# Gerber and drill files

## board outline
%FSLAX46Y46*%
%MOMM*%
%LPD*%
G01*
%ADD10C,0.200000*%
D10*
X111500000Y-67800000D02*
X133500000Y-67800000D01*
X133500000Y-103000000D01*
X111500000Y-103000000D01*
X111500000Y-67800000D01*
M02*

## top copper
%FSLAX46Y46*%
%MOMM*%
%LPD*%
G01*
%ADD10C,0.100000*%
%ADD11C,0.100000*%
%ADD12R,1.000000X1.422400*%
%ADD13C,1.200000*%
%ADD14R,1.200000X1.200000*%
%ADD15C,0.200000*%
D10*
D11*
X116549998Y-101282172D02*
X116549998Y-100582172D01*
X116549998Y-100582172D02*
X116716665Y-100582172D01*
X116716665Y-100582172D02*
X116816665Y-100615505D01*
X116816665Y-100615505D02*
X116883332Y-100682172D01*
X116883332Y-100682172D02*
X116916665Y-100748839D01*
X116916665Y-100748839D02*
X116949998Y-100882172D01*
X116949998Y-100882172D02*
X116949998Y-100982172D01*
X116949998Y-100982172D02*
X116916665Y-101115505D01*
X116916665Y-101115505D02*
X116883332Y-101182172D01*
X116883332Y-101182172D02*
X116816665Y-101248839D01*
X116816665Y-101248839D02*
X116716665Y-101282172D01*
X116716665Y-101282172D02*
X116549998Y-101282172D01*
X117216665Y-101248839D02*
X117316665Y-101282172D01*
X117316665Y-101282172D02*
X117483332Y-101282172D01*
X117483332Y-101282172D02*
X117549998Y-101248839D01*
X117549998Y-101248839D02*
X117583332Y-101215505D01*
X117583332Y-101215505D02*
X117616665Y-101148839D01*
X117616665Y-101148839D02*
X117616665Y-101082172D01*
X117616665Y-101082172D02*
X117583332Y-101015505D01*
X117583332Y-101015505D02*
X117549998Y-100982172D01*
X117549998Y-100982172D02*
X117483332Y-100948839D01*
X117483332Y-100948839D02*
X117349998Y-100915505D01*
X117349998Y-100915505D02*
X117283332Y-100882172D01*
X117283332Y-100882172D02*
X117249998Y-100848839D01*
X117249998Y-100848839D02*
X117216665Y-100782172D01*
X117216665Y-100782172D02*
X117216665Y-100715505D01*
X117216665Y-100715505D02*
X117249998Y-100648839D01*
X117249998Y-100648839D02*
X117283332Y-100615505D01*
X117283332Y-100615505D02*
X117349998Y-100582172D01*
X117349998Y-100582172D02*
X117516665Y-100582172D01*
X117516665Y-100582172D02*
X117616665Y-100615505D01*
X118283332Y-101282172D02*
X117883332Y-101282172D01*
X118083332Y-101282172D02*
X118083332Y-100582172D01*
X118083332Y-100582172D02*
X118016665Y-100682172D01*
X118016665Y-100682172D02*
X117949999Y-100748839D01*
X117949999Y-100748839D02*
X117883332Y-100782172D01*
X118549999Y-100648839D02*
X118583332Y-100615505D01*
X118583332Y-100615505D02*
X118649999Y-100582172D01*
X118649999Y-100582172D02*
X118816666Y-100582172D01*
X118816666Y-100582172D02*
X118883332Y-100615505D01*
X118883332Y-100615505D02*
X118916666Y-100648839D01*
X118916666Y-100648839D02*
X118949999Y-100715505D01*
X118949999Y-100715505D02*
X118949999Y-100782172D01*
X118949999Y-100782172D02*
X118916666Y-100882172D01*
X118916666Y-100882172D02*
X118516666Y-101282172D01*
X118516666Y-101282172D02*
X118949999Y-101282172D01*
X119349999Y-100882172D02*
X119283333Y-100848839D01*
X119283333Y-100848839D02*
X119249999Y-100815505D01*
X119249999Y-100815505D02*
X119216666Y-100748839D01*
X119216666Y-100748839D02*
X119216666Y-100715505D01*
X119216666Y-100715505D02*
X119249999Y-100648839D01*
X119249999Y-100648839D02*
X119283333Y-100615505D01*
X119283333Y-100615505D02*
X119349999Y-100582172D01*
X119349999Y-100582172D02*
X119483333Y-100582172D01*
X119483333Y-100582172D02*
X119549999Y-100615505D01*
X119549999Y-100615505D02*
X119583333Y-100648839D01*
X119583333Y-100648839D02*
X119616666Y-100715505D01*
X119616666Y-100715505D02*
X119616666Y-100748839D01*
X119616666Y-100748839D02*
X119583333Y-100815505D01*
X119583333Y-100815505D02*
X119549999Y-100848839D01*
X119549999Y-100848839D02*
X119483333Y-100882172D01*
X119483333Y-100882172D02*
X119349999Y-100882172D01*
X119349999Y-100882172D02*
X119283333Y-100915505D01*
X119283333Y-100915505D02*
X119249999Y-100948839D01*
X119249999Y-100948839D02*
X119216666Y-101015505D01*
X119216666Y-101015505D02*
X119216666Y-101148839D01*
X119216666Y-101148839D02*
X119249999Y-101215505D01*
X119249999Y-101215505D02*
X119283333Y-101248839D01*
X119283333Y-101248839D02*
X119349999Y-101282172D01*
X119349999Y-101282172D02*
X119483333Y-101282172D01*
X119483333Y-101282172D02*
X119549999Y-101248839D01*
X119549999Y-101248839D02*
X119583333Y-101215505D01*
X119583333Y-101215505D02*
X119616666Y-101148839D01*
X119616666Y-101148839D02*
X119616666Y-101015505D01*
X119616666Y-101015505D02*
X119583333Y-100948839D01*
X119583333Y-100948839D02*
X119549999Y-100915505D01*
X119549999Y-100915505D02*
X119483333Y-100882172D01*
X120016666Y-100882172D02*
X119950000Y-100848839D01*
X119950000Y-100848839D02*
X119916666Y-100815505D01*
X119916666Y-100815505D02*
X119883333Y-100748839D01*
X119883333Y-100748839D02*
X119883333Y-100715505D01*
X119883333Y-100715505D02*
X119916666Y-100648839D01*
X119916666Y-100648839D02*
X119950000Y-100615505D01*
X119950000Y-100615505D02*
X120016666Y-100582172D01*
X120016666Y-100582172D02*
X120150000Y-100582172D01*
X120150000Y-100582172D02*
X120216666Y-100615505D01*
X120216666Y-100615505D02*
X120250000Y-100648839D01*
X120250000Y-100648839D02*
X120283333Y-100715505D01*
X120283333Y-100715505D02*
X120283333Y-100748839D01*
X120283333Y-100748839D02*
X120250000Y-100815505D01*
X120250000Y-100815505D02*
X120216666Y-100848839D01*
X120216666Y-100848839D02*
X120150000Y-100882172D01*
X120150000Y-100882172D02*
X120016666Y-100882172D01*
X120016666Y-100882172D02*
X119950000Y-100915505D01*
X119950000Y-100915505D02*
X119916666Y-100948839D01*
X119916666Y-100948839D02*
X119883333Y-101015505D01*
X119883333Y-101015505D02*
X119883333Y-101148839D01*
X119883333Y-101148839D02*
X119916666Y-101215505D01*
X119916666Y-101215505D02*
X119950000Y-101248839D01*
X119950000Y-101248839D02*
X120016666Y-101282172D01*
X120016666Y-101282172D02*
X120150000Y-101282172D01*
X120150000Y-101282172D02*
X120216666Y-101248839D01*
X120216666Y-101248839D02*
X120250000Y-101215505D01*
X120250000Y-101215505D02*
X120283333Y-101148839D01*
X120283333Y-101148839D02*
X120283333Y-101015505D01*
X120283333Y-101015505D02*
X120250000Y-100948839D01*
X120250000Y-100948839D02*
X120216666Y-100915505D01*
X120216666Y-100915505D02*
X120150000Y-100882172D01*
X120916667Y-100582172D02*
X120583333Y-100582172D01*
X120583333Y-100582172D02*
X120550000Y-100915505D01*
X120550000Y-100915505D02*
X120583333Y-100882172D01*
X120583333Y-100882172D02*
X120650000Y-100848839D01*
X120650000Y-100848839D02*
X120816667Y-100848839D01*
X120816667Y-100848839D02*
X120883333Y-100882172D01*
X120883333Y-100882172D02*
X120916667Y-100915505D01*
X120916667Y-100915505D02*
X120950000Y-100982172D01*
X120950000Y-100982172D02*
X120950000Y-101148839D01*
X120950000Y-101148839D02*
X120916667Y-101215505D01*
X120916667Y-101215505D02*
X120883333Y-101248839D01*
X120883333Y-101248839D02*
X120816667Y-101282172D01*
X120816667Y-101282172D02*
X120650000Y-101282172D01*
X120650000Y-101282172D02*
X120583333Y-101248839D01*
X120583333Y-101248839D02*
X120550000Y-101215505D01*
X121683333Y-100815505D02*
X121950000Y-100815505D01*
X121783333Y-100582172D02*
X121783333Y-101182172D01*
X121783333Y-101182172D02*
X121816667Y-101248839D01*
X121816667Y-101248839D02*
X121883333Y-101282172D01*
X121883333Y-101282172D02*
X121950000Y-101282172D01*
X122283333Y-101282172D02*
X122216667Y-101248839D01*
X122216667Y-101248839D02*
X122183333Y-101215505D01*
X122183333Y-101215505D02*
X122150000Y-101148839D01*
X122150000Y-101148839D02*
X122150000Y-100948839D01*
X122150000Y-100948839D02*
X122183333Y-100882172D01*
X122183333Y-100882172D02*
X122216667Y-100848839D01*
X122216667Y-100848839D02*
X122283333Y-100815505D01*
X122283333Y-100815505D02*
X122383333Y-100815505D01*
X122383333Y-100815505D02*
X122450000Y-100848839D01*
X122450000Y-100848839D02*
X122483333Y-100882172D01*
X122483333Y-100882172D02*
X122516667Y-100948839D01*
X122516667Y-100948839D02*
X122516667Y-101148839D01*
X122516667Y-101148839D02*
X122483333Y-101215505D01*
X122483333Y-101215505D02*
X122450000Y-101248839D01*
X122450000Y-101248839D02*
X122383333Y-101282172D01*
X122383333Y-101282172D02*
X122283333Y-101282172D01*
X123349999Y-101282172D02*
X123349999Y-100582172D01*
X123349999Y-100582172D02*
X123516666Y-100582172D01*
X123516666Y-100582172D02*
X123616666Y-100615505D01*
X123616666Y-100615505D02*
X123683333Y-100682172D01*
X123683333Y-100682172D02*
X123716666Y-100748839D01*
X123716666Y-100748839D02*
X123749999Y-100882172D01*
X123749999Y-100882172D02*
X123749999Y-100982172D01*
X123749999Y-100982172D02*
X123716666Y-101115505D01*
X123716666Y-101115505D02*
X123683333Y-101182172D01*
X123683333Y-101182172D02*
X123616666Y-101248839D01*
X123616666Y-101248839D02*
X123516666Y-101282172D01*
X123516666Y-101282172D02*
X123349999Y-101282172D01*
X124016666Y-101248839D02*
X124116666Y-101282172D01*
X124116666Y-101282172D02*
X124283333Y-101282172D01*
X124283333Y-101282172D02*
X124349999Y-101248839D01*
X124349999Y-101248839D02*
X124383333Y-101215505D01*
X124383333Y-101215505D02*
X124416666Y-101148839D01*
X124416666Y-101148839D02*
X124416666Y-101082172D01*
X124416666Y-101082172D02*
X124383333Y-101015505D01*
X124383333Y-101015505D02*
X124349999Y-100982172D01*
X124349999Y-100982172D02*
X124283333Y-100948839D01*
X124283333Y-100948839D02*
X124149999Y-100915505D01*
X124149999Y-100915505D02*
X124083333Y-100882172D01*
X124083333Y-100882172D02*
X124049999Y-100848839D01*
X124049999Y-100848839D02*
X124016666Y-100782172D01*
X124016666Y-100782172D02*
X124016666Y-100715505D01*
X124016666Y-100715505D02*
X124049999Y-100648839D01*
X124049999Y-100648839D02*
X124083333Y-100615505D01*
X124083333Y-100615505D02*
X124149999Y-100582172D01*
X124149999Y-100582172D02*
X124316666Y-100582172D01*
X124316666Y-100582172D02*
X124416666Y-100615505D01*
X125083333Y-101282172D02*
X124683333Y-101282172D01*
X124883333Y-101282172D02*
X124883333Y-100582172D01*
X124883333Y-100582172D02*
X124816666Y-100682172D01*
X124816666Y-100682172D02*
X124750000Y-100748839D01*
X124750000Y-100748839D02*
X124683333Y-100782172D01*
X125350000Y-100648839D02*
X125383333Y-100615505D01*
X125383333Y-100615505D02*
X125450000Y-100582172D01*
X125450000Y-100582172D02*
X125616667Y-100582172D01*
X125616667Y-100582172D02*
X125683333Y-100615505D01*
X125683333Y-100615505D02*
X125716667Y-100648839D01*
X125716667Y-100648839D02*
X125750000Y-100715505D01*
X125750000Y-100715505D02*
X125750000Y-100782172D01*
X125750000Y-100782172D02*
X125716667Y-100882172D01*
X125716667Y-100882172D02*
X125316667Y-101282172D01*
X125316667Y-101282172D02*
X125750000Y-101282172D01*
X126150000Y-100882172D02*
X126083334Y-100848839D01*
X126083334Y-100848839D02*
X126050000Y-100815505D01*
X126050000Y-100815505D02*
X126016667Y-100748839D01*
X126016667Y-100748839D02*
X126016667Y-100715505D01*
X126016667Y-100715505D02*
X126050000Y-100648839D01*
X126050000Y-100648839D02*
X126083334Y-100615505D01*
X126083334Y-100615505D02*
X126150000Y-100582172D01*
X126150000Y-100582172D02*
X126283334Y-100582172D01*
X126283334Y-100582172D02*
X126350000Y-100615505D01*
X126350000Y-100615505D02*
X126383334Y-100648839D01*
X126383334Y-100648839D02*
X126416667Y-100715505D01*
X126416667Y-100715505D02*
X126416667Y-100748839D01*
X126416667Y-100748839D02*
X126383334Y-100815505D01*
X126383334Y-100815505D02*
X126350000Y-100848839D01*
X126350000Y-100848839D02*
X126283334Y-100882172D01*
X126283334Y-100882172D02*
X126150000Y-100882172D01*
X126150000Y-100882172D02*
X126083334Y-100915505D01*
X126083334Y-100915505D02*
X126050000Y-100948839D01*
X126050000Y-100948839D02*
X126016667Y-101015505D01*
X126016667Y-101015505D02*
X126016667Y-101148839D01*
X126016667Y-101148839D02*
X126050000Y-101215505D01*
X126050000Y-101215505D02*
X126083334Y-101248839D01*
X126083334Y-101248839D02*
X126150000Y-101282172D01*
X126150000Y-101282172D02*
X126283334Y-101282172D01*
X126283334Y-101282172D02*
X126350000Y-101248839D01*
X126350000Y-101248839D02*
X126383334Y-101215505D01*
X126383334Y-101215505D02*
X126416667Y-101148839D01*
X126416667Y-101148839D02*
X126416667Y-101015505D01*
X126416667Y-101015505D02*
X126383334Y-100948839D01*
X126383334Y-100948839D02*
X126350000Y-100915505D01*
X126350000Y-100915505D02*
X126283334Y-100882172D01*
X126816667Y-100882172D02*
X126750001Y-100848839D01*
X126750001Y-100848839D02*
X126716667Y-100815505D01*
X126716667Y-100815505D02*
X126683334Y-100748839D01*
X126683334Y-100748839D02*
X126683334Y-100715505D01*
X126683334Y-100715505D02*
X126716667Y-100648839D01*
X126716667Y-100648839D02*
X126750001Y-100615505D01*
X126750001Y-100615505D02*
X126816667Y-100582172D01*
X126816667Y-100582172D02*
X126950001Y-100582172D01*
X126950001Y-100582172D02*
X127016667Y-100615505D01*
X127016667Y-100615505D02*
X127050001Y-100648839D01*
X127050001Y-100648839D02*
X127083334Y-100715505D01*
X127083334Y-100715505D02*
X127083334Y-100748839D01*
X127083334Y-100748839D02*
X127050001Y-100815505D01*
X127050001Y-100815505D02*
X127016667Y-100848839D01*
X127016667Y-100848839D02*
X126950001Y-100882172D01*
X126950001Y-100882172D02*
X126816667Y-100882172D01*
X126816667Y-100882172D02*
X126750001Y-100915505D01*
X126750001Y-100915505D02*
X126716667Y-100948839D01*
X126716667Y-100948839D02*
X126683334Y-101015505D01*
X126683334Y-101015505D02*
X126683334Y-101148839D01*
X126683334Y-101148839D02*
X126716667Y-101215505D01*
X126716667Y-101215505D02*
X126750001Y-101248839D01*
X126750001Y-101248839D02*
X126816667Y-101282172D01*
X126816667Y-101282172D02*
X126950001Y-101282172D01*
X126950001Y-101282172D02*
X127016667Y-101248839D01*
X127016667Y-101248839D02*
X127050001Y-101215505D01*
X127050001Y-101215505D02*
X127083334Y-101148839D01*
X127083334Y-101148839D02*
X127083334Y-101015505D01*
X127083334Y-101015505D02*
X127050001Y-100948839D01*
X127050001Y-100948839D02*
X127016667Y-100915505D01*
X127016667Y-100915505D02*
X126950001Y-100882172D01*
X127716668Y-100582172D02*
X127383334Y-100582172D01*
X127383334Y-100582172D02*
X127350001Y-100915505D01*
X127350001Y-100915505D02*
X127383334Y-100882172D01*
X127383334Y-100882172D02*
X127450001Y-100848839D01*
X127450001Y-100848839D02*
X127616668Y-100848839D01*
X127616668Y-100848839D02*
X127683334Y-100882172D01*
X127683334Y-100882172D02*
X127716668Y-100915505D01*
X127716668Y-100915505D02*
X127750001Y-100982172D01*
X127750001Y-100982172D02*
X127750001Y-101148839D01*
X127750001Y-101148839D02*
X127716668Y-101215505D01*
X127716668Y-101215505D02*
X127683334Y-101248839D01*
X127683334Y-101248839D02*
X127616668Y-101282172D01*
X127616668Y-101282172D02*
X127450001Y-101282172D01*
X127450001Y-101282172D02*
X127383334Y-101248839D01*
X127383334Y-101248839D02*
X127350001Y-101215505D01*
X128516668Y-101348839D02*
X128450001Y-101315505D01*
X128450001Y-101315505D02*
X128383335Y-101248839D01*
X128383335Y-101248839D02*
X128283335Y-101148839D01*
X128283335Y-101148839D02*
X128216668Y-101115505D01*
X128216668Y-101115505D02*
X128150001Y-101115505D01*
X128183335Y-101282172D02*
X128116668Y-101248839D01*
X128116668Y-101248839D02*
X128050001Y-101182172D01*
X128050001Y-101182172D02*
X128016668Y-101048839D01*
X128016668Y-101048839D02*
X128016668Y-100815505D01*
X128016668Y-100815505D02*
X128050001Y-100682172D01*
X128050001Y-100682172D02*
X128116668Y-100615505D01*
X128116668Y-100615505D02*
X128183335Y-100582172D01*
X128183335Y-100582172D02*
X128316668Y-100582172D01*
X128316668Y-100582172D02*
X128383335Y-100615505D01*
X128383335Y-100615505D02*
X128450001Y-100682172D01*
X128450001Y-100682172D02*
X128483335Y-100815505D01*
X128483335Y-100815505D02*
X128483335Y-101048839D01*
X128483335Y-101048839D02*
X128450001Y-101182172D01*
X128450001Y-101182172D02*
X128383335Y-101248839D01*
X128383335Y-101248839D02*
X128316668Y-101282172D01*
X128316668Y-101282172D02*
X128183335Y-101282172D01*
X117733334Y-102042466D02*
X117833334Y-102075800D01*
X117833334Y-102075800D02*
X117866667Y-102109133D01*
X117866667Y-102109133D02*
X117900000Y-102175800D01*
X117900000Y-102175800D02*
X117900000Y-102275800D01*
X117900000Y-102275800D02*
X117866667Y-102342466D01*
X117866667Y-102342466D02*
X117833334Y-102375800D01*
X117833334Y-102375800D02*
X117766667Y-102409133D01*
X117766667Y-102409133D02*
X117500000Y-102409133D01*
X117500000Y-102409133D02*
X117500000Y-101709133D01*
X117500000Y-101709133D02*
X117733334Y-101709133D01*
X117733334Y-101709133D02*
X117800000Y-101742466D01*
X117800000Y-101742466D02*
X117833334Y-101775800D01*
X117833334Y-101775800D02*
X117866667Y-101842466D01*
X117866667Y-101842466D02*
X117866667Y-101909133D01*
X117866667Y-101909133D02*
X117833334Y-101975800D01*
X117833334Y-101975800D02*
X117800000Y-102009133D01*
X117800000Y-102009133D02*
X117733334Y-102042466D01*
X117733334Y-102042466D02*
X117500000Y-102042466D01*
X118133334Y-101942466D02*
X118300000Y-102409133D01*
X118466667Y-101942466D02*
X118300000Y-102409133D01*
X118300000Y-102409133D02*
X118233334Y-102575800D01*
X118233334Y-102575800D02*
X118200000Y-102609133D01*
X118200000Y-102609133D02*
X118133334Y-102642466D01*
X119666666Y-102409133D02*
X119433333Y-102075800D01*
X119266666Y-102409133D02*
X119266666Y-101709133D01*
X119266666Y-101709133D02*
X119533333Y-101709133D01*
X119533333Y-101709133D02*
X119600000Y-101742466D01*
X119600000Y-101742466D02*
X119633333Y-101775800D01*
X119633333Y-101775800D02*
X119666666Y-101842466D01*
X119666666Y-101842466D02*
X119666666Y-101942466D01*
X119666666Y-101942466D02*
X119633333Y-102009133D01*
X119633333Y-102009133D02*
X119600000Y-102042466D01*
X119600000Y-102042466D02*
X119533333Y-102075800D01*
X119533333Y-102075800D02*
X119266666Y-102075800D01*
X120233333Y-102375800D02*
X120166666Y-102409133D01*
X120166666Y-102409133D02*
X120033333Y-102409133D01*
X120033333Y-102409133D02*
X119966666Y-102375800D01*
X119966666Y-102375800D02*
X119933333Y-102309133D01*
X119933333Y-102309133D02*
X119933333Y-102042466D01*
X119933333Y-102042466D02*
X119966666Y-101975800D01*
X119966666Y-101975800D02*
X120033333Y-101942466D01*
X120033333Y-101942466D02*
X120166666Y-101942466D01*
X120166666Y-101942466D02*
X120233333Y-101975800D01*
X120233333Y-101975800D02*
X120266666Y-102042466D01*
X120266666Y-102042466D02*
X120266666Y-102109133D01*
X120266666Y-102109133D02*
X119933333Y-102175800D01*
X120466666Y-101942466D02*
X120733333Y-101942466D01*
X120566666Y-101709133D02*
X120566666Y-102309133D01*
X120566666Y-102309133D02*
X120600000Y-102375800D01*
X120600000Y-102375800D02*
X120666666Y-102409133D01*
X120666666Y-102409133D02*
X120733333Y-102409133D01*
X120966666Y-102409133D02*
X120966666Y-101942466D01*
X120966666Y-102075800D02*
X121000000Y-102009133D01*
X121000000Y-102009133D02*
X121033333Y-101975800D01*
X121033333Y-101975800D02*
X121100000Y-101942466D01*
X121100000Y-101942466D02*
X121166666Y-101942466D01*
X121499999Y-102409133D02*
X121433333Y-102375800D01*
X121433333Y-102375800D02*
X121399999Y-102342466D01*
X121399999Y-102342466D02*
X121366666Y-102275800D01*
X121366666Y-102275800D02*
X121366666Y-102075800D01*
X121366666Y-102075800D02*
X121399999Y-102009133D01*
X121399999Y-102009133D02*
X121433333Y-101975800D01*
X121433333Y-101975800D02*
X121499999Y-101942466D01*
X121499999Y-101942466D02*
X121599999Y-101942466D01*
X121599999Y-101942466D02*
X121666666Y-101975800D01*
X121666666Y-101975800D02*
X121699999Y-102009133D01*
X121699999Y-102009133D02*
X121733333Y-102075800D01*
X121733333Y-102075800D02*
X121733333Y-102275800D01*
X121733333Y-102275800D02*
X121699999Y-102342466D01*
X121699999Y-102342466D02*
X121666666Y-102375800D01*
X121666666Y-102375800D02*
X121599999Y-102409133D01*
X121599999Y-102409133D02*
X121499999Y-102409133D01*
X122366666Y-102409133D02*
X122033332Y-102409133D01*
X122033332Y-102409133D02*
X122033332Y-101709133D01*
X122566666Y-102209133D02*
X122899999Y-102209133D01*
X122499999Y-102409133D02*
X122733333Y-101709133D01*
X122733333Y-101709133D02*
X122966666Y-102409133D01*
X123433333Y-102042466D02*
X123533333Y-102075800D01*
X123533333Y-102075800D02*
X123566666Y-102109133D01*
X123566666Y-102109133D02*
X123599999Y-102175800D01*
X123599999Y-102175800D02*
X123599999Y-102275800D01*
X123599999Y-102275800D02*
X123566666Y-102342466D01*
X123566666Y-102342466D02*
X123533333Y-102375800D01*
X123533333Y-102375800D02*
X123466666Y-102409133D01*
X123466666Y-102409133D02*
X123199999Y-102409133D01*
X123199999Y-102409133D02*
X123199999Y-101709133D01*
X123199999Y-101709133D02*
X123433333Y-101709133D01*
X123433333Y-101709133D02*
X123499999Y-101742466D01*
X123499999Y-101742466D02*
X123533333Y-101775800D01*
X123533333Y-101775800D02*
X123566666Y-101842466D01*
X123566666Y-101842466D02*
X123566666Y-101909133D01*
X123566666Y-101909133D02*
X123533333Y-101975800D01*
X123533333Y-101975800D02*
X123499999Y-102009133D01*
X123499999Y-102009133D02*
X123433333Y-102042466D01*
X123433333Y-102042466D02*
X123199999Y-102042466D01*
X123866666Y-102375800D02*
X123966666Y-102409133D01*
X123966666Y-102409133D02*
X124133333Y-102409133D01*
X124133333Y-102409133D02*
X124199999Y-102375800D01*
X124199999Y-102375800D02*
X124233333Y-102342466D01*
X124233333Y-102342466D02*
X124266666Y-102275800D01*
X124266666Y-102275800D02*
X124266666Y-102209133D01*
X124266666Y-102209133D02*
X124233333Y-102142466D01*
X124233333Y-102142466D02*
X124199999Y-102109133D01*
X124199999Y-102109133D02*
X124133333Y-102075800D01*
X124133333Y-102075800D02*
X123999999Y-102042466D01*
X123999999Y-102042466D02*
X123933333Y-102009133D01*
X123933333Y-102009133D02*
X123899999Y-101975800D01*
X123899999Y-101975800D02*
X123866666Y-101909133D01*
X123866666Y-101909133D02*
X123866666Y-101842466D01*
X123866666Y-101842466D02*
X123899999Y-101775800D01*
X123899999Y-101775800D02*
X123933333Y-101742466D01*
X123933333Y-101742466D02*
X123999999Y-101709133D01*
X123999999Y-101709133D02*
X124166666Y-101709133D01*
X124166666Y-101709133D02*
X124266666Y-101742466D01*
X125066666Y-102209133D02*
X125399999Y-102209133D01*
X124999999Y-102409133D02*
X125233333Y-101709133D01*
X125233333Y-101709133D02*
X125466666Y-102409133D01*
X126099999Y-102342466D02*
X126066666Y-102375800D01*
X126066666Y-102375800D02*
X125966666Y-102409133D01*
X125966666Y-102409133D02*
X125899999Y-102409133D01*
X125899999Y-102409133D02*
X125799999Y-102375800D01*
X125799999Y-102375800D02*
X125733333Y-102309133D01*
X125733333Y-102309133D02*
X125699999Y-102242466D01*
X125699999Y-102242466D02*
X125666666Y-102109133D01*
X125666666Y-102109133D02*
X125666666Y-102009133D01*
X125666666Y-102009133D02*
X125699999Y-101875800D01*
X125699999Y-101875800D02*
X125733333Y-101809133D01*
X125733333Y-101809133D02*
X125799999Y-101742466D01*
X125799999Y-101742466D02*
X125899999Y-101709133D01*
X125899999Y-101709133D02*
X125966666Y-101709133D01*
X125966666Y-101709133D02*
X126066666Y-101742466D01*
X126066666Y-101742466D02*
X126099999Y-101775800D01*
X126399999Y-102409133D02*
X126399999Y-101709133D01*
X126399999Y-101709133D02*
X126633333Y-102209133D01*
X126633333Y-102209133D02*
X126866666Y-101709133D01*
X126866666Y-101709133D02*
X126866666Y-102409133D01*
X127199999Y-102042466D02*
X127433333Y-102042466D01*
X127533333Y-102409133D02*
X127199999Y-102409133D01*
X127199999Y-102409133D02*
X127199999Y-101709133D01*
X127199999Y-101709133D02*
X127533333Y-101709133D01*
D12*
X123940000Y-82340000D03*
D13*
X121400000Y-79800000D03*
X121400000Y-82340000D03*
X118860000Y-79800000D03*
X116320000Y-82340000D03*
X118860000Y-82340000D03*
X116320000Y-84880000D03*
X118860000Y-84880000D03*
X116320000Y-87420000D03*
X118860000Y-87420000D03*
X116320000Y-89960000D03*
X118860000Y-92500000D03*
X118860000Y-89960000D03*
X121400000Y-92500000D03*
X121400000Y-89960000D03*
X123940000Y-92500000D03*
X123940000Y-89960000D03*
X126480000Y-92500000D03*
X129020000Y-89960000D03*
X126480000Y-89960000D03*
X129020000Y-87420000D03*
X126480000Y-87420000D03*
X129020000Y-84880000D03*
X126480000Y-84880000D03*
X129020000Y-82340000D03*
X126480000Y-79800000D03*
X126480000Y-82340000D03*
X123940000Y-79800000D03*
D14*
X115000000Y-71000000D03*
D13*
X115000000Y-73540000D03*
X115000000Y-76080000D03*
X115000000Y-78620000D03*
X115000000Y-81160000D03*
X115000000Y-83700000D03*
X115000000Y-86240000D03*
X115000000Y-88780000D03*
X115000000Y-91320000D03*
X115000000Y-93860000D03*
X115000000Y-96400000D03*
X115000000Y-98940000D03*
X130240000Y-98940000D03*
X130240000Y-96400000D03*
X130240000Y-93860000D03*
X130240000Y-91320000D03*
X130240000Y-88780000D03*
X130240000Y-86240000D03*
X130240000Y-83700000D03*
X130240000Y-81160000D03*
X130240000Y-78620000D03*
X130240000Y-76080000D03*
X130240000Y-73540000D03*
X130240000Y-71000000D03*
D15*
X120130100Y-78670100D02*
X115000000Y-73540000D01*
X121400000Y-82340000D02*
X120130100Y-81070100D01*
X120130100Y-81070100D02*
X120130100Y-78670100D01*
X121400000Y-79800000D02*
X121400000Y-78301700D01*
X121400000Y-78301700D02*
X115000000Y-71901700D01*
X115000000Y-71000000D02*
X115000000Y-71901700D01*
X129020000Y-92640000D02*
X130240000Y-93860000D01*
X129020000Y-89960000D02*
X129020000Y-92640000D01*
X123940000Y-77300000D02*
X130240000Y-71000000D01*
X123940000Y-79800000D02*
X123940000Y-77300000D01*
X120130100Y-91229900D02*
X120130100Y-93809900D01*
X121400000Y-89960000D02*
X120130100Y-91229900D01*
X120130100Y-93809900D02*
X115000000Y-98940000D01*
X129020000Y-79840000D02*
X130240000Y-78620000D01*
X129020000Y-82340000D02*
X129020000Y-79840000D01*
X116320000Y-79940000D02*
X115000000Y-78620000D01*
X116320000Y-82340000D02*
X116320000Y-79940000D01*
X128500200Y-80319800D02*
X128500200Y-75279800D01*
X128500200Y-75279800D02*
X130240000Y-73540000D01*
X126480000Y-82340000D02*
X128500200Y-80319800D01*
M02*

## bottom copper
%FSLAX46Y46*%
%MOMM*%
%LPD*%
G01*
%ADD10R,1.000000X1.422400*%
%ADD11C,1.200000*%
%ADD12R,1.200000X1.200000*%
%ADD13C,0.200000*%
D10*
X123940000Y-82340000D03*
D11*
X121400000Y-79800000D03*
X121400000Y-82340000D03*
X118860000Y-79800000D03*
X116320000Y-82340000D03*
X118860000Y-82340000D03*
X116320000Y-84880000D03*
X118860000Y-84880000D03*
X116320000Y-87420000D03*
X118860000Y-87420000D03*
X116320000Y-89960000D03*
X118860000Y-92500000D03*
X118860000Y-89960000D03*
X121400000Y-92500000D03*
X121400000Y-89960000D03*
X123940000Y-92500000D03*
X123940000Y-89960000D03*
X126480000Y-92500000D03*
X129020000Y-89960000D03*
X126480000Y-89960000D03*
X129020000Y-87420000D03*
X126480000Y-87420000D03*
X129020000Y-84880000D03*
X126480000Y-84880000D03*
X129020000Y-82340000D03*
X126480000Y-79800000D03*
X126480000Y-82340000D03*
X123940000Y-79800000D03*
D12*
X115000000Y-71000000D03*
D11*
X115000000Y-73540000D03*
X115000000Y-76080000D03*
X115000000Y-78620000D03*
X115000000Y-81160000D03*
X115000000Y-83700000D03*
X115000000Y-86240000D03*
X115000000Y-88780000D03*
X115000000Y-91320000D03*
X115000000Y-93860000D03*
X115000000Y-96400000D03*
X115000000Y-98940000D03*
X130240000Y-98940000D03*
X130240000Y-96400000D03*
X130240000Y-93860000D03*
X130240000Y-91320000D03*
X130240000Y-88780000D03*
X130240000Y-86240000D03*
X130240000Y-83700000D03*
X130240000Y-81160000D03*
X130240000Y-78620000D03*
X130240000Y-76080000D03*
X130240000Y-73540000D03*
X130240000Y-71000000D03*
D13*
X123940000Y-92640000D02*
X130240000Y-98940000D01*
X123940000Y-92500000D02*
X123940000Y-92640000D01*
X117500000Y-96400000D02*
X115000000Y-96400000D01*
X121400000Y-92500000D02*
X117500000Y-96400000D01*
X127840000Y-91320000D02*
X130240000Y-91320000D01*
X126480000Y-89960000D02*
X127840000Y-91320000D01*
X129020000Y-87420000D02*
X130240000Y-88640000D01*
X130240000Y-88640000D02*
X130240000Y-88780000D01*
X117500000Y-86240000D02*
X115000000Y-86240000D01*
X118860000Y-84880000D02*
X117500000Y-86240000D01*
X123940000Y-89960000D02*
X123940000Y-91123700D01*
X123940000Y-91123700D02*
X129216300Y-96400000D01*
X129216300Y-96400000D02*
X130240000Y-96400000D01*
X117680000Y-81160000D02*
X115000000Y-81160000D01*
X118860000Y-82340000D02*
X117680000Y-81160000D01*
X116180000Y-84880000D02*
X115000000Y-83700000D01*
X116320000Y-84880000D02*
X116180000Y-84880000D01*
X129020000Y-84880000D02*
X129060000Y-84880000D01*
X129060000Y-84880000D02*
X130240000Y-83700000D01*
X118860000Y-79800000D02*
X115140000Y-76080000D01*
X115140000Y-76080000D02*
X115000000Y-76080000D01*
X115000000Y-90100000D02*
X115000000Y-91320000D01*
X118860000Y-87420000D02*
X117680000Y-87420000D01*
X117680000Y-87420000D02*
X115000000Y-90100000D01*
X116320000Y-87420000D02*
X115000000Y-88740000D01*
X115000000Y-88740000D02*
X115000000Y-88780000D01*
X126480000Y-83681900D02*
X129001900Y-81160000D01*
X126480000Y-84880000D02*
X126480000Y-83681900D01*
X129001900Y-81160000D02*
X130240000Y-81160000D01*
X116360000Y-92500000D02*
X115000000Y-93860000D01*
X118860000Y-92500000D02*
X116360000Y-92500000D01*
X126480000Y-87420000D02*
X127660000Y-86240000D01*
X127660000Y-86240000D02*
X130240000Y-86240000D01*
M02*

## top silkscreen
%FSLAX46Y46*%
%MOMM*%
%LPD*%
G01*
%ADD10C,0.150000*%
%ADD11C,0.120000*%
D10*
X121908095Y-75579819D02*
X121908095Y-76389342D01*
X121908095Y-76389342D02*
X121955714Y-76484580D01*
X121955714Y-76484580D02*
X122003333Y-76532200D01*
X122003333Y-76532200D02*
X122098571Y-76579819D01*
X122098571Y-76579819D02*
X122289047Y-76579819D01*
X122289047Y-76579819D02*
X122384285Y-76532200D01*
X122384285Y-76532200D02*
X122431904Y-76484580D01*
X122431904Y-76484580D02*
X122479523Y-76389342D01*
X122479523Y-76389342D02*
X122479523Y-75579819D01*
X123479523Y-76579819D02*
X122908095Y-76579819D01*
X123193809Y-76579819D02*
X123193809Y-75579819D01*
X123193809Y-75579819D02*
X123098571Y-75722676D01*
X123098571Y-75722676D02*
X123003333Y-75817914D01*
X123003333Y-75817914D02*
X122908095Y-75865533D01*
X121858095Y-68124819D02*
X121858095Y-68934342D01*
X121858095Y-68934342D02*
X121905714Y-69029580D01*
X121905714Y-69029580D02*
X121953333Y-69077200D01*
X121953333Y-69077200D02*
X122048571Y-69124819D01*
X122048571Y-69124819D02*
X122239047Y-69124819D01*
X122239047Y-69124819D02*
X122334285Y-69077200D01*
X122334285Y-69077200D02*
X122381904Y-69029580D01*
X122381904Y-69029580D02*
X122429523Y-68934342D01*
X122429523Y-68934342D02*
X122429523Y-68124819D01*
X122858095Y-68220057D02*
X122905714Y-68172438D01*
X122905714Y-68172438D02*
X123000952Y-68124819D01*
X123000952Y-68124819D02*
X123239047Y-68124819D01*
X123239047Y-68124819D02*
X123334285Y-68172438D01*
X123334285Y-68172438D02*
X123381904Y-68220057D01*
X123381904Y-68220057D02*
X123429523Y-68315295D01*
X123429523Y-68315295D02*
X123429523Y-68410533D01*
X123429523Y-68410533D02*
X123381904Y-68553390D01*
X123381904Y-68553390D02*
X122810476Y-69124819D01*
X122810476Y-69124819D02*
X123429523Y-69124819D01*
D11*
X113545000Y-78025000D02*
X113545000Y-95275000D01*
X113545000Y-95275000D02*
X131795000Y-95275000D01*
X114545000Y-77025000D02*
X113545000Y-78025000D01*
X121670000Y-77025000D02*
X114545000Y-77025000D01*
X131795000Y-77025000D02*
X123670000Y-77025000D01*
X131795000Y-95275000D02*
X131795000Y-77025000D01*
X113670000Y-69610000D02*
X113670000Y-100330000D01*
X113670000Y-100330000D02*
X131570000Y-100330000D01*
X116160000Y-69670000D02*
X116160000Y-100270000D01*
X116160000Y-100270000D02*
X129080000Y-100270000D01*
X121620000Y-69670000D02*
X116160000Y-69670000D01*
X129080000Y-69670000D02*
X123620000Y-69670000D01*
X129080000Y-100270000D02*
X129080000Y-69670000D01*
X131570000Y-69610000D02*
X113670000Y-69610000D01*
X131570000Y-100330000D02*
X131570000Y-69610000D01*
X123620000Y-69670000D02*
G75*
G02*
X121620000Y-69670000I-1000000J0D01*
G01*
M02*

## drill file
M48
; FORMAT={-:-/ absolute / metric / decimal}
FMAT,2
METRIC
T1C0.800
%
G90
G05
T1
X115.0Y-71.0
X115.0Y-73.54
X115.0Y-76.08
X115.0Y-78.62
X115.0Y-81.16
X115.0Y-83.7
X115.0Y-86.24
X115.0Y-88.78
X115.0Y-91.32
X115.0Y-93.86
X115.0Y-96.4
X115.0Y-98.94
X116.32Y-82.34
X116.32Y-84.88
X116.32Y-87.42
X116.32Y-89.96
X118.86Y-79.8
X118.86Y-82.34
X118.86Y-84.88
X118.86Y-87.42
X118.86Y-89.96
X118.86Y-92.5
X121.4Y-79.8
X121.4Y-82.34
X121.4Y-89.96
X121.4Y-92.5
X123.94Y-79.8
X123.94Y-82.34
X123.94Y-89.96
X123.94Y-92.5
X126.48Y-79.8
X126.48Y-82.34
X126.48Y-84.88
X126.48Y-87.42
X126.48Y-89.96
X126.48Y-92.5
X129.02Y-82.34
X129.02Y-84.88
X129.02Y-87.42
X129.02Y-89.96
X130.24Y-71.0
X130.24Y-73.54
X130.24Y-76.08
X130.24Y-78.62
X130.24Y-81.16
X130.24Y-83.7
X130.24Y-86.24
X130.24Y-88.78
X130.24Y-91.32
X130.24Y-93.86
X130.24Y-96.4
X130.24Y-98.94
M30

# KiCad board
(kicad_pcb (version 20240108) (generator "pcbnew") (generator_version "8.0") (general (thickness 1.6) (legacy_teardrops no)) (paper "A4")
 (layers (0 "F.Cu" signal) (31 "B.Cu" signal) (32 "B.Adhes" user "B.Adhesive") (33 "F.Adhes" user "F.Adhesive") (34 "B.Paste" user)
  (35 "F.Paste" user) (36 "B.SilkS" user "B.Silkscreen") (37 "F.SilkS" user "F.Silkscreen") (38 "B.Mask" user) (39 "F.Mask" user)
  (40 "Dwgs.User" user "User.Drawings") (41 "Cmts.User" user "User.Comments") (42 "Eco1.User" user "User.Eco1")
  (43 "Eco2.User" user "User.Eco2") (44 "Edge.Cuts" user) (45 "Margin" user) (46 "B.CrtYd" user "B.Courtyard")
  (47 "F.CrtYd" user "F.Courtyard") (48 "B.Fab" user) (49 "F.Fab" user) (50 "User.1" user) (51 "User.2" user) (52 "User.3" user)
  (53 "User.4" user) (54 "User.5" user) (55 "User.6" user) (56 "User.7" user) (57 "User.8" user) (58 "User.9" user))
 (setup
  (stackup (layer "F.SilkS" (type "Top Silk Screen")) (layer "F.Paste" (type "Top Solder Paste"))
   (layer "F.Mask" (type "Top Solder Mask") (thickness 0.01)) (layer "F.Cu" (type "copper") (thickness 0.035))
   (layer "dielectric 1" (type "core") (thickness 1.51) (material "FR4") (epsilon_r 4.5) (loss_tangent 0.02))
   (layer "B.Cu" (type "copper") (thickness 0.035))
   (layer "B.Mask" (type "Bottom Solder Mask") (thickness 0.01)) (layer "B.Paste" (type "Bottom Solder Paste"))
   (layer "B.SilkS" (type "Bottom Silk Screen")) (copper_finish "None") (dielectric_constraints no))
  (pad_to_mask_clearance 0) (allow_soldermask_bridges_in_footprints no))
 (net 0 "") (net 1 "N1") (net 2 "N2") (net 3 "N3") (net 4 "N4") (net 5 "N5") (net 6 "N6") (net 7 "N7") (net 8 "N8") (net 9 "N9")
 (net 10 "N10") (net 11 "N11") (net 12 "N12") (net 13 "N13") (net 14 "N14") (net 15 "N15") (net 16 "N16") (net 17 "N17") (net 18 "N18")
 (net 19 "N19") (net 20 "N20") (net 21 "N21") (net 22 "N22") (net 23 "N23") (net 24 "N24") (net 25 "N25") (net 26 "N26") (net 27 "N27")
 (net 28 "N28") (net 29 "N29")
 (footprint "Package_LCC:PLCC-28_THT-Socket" (layer "F.Cu") (at 123.94 82.34)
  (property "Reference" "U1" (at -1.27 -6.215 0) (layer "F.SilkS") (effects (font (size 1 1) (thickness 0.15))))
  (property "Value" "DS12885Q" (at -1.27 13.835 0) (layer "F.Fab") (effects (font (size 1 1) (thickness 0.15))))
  (fp_line (start -10.395 -4.315) (end -10.395 12.935) (stroke (width 0.12) (type solid)) (layer "F.SilkS"))
  (fp_line (start -10.395 12.935) (end 7.855 12.935) (stroke (width 0.12) (type solid)) (layer "F.SilkS"))
  (fp_line (start -9.395 -5.315) (end -10.395 -4.315) (stroke (width 0.12) (type solid)) (layer "F.SilkS"))
  (fp_line (start -2.27 -5.315) (end -9.395 -5.315) (stroke (width 0.12) (type solid)) (layer "F.SilkS"))
  (fp_line (start 7.855 -5.315) (end -0.27 -5.315) (stroke (width 0.12) (type solid)) (layer "F.SilkS"))
  (fp_line (start 7.855 12.935) (end 7.855 -5.315) (stroke (width 0.12) (type solid)) (layer "F.SilkS"))
  (pad "1" thru_hole rect (at 0 0) (size 1 1.4224) (drill 0.8) (layers "*.Cu" "*.Mask") (remove_unused_layers no) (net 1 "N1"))
  (pad "2" thru_hole circle (at -2.54 -2.54) (size 1.2 1) (drill 0.8) (layers "*.Cu" "*.Mask") (remove_unused_layers no) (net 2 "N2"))
  (pad "3" thru_hole circle (at -2.54 0) (size 1.2 1) (drill 0.8) (layers "*.Cu" "*.Mask") (remove_unused_layers no) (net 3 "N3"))
  (pad "4" thru_hole circle (at -5.08 -2.54) (size 1.2 1) (drill 0.8) (layers "*.Cu" "*.Mask") (remove_unused_layers no) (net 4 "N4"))
  (pad "5" thru_hole circle (at -7.62 0) (size 1.2 1) (drill 0.8) (layers "*.Cu" "*.Mask") (remove_unused_layers no) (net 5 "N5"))
  (pad "6" thru_hole circle (at -5.08 0) (size 1.2 1) (drill 0.8) (layers "*.Cu" "*.Mask") (remove_unused_layers no) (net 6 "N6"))
  (pad "7" thru_hole circle (at -7.62 2.54) (size 1.2 1) (drill 0.8) (layers "*.Cu" "*.Mask") (remove_unused_layers no) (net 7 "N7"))
  (pad "8" thru_hole circle (at -5.08 2.54) (size 1.2 1) (drill 0.8) (layers "*.Cu" "*.Mask") (remove_unused_layers no) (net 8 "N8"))
  (pad "9" thru_hole circle (at -7.62 5.08) (size 1.2 1) (drill 0.8) (layers "*.Cu" "*.Mask") (remove_unused_layers no) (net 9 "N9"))
  (pad "10" thru_hole circle (at -5.08 5.08) (size 1.2 1) (drill 0.8) (layers "*.Cu" "*.Mask") (remove_unused_layers no) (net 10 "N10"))
  (pad "11" thru_hole circle (at -7.62 7.62) (size 1.2 1) (drill 0.8) (layers "*.Cu" "*.Mask") (remove_unused_layers no) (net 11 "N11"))
  (pad "12" thru_hole circle (at -5.08 10.16) (size 1.2 1) (drill 0.8) (layers "*.Cu" "*.Mask") (remove_unused_layers no) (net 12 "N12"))
  (pad "13" thru_hole circle (at -5.08 7.62) (size 1.2 1) (drill 0.8) (layers "*.Cu" "*.Mask") (remove_unused_layers no) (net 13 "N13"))
  (pad "14" thru_hole circle (at -2.54 10.16) (size 1.2 1) (drill 0.8) (layers "*.Cu" "*.Mask") (remove_unused_layers no) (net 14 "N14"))
  (pad "15" thru_hole circle (at -2.54 7.62) (size 1.2 1) (drill 0.8) (layers "*.Cu" "*.Mask") (remove_unused_layers no) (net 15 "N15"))
  (pad "16" thru_hole circle (at 0 10.16) (size 1.2 1) (drill 0.8) (layers "*.Cu" "*.Mask") (remove_unused_layers no) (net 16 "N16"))
  (pad "17" thru_hole circle (at 0 7.62) (size 1.2 1) (drill 0.8) (layers "*.Cu" "*.Mask") (remove_unused_layers no) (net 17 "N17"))
  (pad "18" thru_hole circle (at 2.54 10.16) (size 1.2 1) (drill 0.8) (layers "*.Cu" "*.Mask") (remove_unused_layers no) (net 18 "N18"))
  (pad "19" thru_hole circle (at 5.08 7.62) (size 1.2 1) (drill 0.8) (layers "*.Cu" "*.Mask") (remove_unused_layers no) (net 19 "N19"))
  (pad "20" thru_hole circle (at 2.54 7.62) (size 1.2 1) (drill 0.8) (layers "*.Cu" "*.Mask") (remove_unused_layers no) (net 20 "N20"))
  (pad "21" thru_hole circle (at 5.08 5.08) (size 1.2 1) (drill 0.8) (layers "*.Cu" "*.Mask") (remove_unused_layers no) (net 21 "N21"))
  (pad "22" thru_hole circle (at 2.54 5.08) (size 1.2 1) (drill 0.8) (layers "*.Cu" "*.Mask") (remove_unused_layers no) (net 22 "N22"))
  (pad "23" thru_hole circle (at 5.08 2.54) (size 1.2 1) (drill 0.8) (layers "*.Cu" "*.Mask") (remove_unused_layers no) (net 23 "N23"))
  (pad "24" thru_hole circle (at 2.54 2.54) (size 1.2 1) (drill 0.8) (layers "*.Cu" "*.Mask") (remove_unused_layers no) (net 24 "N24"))
  (pad "25" thru_hole circle (at 5.08 0) (size 1.2 1) (drill 0.8) (layers "*.Cu" "*.Mask") (remove_unused_layers no) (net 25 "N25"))
  (pad "26" thru_hole circle (at 2.54 -2.54) (size 1.2 1) (drill 0.8) (layers "*.Cu" "*.Mask") (remove_unused_layers no) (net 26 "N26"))
  (pad "27" thru_hole circle (at 2.54 0) (size 1.2 1) (drill 0.8) (layers "*.Cu" "*.Mask") (remove_unused_layers no) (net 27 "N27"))
  (pad "28" thru_hole circle (at 0 -2.54) (size 1.2 1) (drill 0.8) (layers "*.Cu" "*.Mask") (remove_unused_layers no) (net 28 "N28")))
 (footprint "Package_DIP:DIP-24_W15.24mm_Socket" (layer "F.Cu") (at 115 71)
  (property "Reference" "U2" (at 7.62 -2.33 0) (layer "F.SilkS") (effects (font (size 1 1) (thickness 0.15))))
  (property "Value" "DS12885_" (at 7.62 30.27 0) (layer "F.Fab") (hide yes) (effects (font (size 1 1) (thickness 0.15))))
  (fp_line (start -1.33 -1.39) (end -1.33 29.33) (stroke (width 0.12) (type solid)) (layer "F.SilkS"))
  (fp_line (start -1.33 29.33) (end 16.57 29.33) (stroke (width 0.12) (type solid)) (layer "F.SilkS"))
  (fp_line (start 1.16 -1.33) (end 1.16 29.27) (stroke (width 0.12) (type solid)) (layer "F.SilkS"))
  (fp_line (start 1.16 29.27) (end 14.08 29.27) (stroke (width 0.12) (type solid)) (layer "F.SilkS"))
  (fp_line (start 6.62 -1.33) (end 1.16 -1.33) (stroke (width 0.12) (type solid)) (layer "F.SilkS"))
  (fp_line (start 14.08 -1.33) (end 8.62 -1.33) (stroke (width 0.12) (type solid)) (layer "F.SilkS"))
  (fp_line (start 14.08 29.27) (end 14.08 -1.33) (stroke (width 0.12) (type solid)) (layer "F.SilkS"))
  (fp_line (start 16.57 -1.39) (end -1.33 -1.39) (stroke (width 0.12) (type solid)) (layer "F.SilkS"))
  (fp_line (start 16.57 29.33) (end 16.57 -1.39) (stroke (width 0.12) (type solid)) (layer "F.SilkS"))
  (fp_arc (start 8.62 -1.33) (mid 7.62 -0.33) (end 6.62 -1.33) (stroke (width 0.12) (type solid)) (layer "F.SilkS"))
  (pad "1" thru_hole rect (at 0 0) (size 1.2 1.2) (drill 0.8) (layers "*.Cu" "*.Mask") (remove_unused_layers no) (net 2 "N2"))
  (pad "2" thru_hole circle (at 0 2.54) (size 1.2 1) (drill 0.8) (layers "*.Cu" "*.Mask") (remove_unused_layers no) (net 3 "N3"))
  (pad "3" thru_hole circle (at 0 5.08) (size 1.2 1) (drill 0.8) (layers "*.Cu" "*.Mask") (remove_unused_layers no) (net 4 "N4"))
  (pad "4" thru_hole circle (at 0 7.62) (size 1.2 1) (drill 0.8) (layers "*.Cu" "*.Mask") (remove_unused_layers no) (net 5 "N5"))
  (pad "5" thru_hole circle (at 0 10.16) (size 1.2 1) (drill 0.8) (layers "*.Cu" "*.Mask") (remove_unused_layers no) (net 6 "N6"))
  (pad "6" thru_hole circle (at 0 12.7) (size 1.2 1) (drill 0.8) (layers "*.Cu" "*.Mask") (remove_unused_layers no) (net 7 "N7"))
  (pad "7" thru_hole circle (at 0 15.24) (size 1.2 1) (drill 0.8) (layers "*.Cu" "*.Mask") (remove_unused_layers no) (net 8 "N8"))
  (pad "8" thru_hole circle (at 0 17.78) (size 1.2 1) (drill 0.8) (layers "*.Cu" "*.Mask") (remove_unused_layers no) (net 9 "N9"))
  (pad "9" thru_hole circle (at 0 20.32) (size 1.2 1) (drill 0.8) (layers "*.Cu" "*.Mask") (remove_unused_layers no) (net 10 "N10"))
  (pad "10" thru_hole circle (at 0 22.86) (size 1.2 1) (drill 0.8) (layers "*.Cu" "*.Mask") (remove_unused_layers no) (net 12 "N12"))
  (pad "11" thru_hole circle (at 0 25.4) (size 1.2 1) (drill 0.8) (layers "*.Cu" "*.Mask") (remove_unused_layers no) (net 14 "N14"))
  (pad "12" thru_hole circle (at 0 27.94) (size 1.2 1) (drill 0.8) (layers "*.Cu" "*.Mask") (remove_unused_layers no) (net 15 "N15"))
  (pad "13" thru_hole circle (at 15.24 27.94) (size 1.2 1) (drill 0.8) (layers "*.Cu" "*.Mask") (remove_unused_layers no) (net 16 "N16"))
  (pad "14" thru_hole circle (at 15.24 25.4) (size 1.2 1) (drill 0.8) (layers "*.Cu" "*.Mask") (remove_unused_layers no) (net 17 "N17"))
  (pad "15" thru_hole circle (at 15.24 22.86) (size 1.2 1) (drill 0.8) (layers "*.Cu" "*.Mask") (remove_unused_layers no) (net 19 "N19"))
  (pad "16" thru_hole circle (at 15.24 20.32) (size 1.2 1) (drill 0.8) (layers "*.Cu" "*.Mask") (remove_unused_layers no) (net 20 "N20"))
  (pad "17" thru_hole circle (at 15.24 17.78) (size 1.2 1) (drill 0.8) (layers "*.Cu" "*.Mask") (remove_unused_layers no) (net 21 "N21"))
  (pad "18" thru_hole circle (at 15.24 15.24) (size 1.2 1) (drill 0.8) (layers "*.Cu" "*.Mask") (remove_unused_layers no) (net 22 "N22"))
  (pad "19" thru_hole circle (at 15.24 12.7) (size 1.2 1) (drill 0.8) (layers "*.Cu" "*.Mask") (remove_unused_layers no) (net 23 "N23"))
  (pad "20" thru_hole circle (at 15.24 10.16) (size 1.2 1) (drill 0.8) (layers "*.Cu" "*.Mask") (remove_unused_layers no) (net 24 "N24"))
  (pad "21" thru_hole circle (at 15.24 7.62) (size 1.2 1) (drill 0.8) (layers "*.Cu" "*.Mask") (remove_unused_layers no) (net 25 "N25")
   (thermal_bridge_angle 90))
  (pad "22" thru_hole circle (at 15.24 5.08) (size 1.2 1) (drill 0.8) (layers "*.Cu" "*.Mask") (remove_unused_layers no) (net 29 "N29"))
  (pad "23" thru_hole circle (at 15.24 2.54) (size 1.2 1) (drill 0.8) (layers "*.Cu" "*.Mask") (remove_unused_layers no) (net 27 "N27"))
  (pad "24" thru_hole circle (at 15.24 0) (size 1.2 1) (drill 0.8) (layers "*.Cu" "*.Mask") (remove_unused_layers no) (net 28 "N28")))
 (gr_rect (start 111.5 67.8) (end 133.5 103) (stroke (width 0.2) (type default)) (fill none) (layer "Edge.Cuts"))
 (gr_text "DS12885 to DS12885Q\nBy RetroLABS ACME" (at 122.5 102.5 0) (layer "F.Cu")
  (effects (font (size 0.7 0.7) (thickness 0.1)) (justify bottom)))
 (segment (start 123.94 92.64) (end 130.24 98.94) (width 0.2) (layer "B.Cu") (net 16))
 (segment (start 123.94 92.5) (end 123.94 92.64) (width 0.2) (layer "B.Cu") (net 16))
 (segment (start 117.5 96.4) (end 115 96.4) (width 0.2) (layer "B.Cu") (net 14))
 (segment (start 121.4 92.5) (end 117.5 96.4) (width 0.2) (layer "B.Cu") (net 14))
 (segment (start 120.1301 78.6701) (end 115 73.54) (width 0.2) (layer "F.Cu") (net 3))
 (segment (start 121.4 82.34) (end 120.1301 81.0701) (width 0.2) (layer "F.Cu") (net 3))
 (segment (start 120.1301 81.0701) (end 120.1301 78.6701) (width 0.2) (layer "F.Cu") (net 3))
 (segment (start 127.84 91.32) (end 130.24 91.32) (width 0.2) (layer "B.Cu") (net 20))
 (segment (start 126.48 89.96) (end 127.84 91.32) (width 0.2) (layer "B.Cu") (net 20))
 (segment (start 129.02 87.42) (end 130.24 88.64) (width 0.2) (layer "B.Cu") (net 21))
 (segment (start 130.24 88.64) (end 130.24 88.78) (width 0.2) (layer "B.Cu") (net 21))
 (segment (start 121.4 79.8) (end 121.4 78.3017) (width 0.2) (layer "F.Cu") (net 2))
 (segment (start 121.4 78.3017) (end 115 71.9017) (width 0.2) (layer "F.Cu") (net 2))
 (segment (start 115 71) (end 115 71.9017) (width 0.2) (layer "F.Cu") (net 2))
 (segment (start 117.5 86.24) (end 115 86.24) (width 0.2) (layer "B.Cu") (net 8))
 (segment (start 118.86 84.88) (end 117.5 86.24) (width 0.2) (layer "B.Cu") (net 8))
 (segment (start 123.94 89.96) (end 123.94 91.1237) (width 0.2) (layer "B.Cu") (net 17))
 (segment (start 123.94 91.1237) (end 129.2163 96.4) (width 0.2) (layer "B.Cu") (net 17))
 (segment (start 129.2163 96.4) (end 130.24 96.4) (width 0.2) (layer "B.Cu") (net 17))
 (segment (start 117.68 81.16) (end 115 81.16) (width 0.2) (layer "B.Cu") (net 6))
 (segment (start 118.86 82.34) (end 117.68 81.16) (width 0.2) (layer "B.Cu") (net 6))
 (segment (start 116.18 84.88) (end 115 83.7) (width 0.2) (layer "B.Cu") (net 7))
 (segment (start 116.32 84.88) (end 116.18 84.88) (width 0.2) (layer "B.Cu") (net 7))
 (segment (start 129.02 84.88) (end 129.06 84.88) (width 0.2) (layer "B.Cu") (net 23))
 (segment (start 129.06 84.88) (end 130.24 83.7) (width 0.2) (layer "B.Cu") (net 23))
 (segment (start 129.02 92.64) (end 130.24 93.86) (width 0.2) (layer "F.Cu") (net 19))
 (segment (start 129.02 89.96) (end 129.02 92.64) (width 0.2) (layer "F.Cu") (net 19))
 (segment (start 118.86 79.8) (end 115.14 76.08) (width 0.2) (layer "B.Cu") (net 4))
 (segment (start 115.14 76.08) (end 115 76.08) (width 0.2) (layer "B.Cu") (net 4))
 (segment (start 115 90.1) (end 115 91.32) (width 0.2) (layer "B.Cu") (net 10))
 (segment (start 118.86 87.42) (end 117.68 87.42) (width 0.2) (layer "B.Cu") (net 10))
 (segment (start 117.68 87.42) (end 115 90.1) (width 0.2) (layer "B.Cu") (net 10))
 (segment (start 116.32 87.42) (end 115 88.74) (width 0.2) (layer "B.Cu") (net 9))
 (segment (start 115 88.74) (end 115 88.78) (width 0.2) (layer "B.Cu") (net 9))
 (segment (start 123.94 77.3) (end 130.24 71) (width 0.2) (layer "F.Cu") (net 28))
 (segment (start 123.94 79.8) (end 123.94 77.3) (width 0.2) (layer "F.Cu") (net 28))
 (segment (start 120.1301 91.2299) (end 120.1301 93.8099) (width 0.2) (layer "F.Cu") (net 15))
 (segment (start 121.4 89.96) (end 120.1301 91.2299) (width 0.2) (layer "F.Cu") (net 15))
 (segment (start 120.1301 93.8099) (end 115 98.94) (width 0.2) (layer "F.Cu") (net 15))
 (segment (start 129.02 79.84) (end 130.24 78.62) (width 0.2) (layer "F.Cu") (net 25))
 (segment (start 129.02 82.34) (end 129.02 79.84) (width 0.2) (layer "F.Cu") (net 25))
 (segment (start 126.48 83.6819) (end 129.0019 81.16) (width 0.2) (layer "B.Cu") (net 24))
 (segment (start 126.48 84.88) (end 126.48 83.6819) (width 0.2) (layer "B.Cu") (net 24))
 (segment (start 129.0019 81.16) (end 130.24 81.16) (width 0.2) (layer "B.Cu") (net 24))
 (segment (start 116.32 79.94) (end 115 78.62) (width 0.2) (layer "F.Cu") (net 5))
 (segment (start 116.32 82.34) (end 116.32 79.94) (width 0.2) (layer "F.Cu") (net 5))
 (segment (start 116.36 92.5) (end 115 93.86) (width 0.2) (layer "B.Cu") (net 12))
 (segment (start 118.86 92.5) (end 116.36 92.5) (width 0.2) (layer "B.Cu") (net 12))
 (segment (start 128.5002 80.3198) (end 128.5002 75.2798) (width 0.2) (layer "F.Cu") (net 27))
 (segment (start 128.5002 75.2798) (end 130.24 73.54) (width 0.2) (layer "F.Cu") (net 27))
 (segment (start 126.48 82.34) (end 128.5002 80.3198) (width 0.2) (layer "F.Cu") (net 27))
 (segment (start 126.48 87.42) (end 127.66 86.24) (width 0.2) (layer "B.Cu") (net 22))
 (segment (start 127.66 86.24) (end 130.24 86.24) (width 0.2) (layer "B.Cu") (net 22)))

